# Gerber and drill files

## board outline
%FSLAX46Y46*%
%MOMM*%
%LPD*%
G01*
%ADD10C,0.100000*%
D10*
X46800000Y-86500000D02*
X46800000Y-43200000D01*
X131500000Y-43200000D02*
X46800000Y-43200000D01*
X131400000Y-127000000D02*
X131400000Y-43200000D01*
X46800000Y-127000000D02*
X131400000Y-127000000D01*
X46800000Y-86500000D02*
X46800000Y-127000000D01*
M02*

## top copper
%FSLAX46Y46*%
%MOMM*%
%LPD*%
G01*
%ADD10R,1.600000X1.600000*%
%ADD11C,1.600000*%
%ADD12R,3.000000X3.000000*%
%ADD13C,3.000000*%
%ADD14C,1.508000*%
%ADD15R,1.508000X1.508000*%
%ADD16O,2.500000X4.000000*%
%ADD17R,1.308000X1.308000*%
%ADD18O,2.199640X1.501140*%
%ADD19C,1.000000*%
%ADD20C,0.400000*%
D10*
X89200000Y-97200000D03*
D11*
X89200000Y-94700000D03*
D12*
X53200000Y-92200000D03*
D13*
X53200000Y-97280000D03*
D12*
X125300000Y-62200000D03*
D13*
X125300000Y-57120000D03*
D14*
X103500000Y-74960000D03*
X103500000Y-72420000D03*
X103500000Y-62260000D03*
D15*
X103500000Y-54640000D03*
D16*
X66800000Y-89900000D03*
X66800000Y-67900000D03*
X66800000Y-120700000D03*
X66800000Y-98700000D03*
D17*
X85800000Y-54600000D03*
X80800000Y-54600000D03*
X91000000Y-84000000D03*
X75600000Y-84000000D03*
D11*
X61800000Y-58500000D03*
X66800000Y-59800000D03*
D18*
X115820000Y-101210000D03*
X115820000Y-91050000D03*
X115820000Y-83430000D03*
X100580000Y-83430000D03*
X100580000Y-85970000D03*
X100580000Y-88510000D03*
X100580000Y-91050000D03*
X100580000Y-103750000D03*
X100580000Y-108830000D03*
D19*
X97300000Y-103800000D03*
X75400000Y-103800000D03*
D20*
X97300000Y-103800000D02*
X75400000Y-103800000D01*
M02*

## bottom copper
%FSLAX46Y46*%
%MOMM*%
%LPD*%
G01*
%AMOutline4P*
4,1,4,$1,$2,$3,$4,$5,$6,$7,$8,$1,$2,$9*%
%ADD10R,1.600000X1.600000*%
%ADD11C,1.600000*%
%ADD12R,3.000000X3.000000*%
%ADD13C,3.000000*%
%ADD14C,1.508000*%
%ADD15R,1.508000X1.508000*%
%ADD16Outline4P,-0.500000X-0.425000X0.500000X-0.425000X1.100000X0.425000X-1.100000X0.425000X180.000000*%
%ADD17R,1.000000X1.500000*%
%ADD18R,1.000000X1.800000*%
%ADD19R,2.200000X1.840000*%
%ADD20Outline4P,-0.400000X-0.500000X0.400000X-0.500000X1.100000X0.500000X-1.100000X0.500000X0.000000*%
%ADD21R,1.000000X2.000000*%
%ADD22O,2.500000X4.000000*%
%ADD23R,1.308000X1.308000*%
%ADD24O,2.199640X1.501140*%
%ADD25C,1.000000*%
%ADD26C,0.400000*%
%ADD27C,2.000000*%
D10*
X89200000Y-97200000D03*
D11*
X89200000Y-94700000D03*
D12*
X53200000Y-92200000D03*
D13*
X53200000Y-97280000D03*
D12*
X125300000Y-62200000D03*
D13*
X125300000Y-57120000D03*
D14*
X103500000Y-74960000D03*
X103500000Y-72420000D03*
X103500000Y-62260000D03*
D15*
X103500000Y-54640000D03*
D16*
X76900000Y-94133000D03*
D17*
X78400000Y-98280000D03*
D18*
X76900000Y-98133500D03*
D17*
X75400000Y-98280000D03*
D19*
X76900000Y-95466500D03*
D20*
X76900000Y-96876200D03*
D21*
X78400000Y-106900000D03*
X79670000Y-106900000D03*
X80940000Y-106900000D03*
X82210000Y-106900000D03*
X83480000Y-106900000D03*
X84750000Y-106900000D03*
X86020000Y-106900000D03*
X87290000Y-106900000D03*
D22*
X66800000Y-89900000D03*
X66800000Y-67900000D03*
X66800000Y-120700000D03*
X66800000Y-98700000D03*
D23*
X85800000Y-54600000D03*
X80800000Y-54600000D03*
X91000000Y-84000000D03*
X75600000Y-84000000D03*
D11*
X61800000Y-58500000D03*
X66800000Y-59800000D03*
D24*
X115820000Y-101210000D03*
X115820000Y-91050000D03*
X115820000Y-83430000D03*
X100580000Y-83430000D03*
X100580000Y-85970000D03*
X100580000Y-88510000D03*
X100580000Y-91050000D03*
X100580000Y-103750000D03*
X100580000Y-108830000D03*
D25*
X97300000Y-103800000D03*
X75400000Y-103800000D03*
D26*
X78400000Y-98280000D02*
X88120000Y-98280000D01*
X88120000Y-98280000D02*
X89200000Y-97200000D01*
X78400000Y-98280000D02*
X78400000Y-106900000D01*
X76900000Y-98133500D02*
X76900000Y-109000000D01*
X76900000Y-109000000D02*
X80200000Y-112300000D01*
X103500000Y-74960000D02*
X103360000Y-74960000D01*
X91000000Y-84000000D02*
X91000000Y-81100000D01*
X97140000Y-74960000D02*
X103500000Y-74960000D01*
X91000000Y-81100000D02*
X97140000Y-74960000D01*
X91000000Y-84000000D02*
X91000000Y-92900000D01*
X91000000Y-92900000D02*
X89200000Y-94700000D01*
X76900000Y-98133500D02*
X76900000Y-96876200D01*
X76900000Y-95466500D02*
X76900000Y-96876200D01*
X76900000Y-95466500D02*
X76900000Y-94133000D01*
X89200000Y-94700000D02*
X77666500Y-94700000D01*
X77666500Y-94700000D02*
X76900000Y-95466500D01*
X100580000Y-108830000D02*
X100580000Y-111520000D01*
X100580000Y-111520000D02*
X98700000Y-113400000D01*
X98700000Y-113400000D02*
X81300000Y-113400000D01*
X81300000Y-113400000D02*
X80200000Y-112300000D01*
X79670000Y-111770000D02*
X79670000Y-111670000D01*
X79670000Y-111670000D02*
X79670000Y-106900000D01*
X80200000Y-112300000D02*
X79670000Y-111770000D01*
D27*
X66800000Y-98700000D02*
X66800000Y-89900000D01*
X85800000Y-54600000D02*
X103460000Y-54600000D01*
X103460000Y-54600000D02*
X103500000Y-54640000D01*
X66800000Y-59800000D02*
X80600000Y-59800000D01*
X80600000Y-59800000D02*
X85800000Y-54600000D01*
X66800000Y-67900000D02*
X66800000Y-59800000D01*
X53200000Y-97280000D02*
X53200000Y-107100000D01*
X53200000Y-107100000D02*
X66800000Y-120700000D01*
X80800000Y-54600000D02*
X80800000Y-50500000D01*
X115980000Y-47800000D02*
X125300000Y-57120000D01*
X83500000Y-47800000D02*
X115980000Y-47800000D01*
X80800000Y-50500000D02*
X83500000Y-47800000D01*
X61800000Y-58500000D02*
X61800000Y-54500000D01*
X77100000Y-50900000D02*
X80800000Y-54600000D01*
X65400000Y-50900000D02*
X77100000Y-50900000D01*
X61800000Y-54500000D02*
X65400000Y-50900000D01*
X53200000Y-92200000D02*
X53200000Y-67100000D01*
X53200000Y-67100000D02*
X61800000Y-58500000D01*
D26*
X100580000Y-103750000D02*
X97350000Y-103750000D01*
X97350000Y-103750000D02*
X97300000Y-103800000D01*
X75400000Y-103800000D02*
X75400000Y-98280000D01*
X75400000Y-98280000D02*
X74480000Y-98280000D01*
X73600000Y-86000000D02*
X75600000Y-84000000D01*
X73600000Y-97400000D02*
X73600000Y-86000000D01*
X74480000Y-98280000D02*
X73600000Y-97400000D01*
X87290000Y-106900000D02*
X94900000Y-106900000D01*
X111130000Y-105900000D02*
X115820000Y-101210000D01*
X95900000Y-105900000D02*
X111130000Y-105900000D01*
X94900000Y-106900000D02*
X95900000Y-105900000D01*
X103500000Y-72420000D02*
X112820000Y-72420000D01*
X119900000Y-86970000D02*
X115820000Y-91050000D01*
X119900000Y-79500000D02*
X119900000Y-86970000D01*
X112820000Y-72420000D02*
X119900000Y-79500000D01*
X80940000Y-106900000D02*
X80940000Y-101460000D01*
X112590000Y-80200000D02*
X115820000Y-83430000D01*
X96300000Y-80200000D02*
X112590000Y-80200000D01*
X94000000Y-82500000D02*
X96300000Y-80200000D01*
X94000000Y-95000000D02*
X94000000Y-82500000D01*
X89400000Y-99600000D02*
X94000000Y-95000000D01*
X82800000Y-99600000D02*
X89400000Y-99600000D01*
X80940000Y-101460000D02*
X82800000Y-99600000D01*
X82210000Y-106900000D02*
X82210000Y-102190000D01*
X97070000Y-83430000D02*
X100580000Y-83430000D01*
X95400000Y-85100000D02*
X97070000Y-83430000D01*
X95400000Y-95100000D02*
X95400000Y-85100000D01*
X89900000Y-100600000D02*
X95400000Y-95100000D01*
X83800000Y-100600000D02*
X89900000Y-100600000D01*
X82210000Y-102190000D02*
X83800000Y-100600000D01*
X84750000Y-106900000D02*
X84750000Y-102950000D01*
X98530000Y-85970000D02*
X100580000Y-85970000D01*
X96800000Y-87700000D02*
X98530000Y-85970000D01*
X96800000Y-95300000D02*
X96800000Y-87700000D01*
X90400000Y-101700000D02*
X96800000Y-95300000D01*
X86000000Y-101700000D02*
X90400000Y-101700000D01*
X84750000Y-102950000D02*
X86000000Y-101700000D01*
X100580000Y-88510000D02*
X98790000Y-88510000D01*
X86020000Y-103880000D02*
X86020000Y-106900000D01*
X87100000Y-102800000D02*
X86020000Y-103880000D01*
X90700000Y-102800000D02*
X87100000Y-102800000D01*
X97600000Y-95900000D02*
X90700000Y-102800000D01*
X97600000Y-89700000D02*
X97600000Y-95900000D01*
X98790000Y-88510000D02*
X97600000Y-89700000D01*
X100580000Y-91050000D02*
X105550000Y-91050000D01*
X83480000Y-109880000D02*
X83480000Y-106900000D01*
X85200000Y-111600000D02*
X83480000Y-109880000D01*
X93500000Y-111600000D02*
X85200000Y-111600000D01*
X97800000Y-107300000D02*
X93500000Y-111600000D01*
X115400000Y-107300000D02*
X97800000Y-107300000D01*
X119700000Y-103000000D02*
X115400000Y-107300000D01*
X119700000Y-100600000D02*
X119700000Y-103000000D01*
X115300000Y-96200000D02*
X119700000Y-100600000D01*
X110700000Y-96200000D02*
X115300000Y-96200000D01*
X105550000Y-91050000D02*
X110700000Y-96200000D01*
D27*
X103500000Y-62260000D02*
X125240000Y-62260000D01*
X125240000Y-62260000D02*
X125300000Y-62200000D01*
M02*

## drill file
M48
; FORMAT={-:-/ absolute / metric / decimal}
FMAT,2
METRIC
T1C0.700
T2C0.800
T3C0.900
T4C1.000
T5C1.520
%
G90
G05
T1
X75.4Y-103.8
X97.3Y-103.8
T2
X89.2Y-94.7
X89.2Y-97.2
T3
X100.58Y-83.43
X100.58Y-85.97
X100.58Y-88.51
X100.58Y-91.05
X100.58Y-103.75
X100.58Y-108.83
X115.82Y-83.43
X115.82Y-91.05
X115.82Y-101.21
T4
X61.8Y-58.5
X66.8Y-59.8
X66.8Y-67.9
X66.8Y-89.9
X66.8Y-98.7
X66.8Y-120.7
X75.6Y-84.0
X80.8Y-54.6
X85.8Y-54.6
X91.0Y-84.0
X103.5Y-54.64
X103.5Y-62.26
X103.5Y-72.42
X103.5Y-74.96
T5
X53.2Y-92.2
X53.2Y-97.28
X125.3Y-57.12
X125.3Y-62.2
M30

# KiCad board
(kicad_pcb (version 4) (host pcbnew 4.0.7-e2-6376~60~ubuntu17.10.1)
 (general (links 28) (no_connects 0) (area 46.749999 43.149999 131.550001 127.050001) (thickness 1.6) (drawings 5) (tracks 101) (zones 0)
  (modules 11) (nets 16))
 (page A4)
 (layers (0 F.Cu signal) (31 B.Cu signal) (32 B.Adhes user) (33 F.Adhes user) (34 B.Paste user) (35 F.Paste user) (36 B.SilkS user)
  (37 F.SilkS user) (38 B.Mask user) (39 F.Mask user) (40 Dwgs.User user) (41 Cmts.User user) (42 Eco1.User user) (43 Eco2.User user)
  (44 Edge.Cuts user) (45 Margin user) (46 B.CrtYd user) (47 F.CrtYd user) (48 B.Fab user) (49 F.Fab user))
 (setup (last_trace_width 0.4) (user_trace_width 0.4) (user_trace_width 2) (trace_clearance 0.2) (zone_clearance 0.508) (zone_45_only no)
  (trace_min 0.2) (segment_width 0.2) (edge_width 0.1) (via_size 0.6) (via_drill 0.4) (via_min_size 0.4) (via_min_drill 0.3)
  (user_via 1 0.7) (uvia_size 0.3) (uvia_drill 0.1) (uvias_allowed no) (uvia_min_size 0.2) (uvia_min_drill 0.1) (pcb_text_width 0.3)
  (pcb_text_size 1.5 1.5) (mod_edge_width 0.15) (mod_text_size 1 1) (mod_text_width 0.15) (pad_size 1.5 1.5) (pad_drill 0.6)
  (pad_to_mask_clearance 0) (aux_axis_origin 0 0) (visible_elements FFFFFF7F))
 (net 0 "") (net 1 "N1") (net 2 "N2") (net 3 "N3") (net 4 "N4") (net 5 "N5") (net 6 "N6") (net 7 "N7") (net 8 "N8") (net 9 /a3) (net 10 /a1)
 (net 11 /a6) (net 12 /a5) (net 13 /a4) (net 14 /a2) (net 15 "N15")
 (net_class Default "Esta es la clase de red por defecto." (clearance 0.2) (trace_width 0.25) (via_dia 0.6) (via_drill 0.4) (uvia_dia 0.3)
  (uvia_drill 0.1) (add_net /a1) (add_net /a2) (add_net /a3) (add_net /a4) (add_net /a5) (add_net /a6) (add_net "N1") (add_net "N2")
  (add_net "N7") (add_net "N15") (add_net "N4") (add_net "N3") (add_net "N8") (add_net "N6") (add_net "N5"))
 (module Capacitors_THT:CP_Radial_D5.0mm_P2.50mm (layer F.Cu) (at 89.2 97.2 90)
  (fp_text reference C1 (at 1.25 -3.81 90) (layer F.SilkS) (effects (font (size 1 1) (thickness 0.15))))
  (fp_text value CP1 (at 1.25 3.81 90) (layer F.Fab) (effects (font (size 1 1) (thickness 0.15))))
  (pad 1 thru_hole rect (at 0 0 90) (size 1.6 1.6) (drill 0.8) (layers *.Cu *.Mask) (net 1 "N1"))
  (pad 2 thru_hole circle (at 2.5 0 90) (size 1.6 1.6) (drill 0.8) (layers *.Cu *.Mask) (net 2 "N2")))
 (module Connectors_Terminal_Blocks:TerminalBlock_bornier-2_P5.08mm (layer F.Cu) (at 53.2 92.2 270)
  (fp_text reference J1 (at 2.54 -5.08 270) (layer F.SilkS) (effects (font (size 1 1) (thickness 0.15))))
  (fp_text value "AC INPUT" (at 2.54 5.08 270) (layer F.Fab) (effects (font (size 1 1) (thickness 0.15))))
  (pad 1 thru_hole rect (at 0 0 270) (size 3 3) (drill 1.52) (layers *.Cu *.Mask) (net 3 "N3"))
  (pad 2 thru_hole circle (at 5.08 0 270) (size 3 3) (drill 1.52) (layers *.Cu *.Mask) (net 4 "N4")))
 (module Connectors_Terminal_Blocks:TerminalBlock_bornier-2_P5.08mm (layer F.Cu) (at 125.3 62.2 90)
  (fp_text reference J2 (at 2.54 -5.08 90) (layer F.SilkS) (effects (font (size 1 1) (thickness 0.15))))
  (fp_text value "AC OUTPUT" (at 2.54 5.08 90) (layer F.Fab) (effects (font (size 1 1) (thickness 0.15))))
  (pad 1 thru_hole rect (at 0 0 90) (size 3 3) (drill 1.52) (layers *.Cu *.Mask) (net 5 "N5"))
  (pad 2 thru_hole circle (at 5.08 0 90) (size 3 3) (drill 1.52) (layers *.Cu *.Mask) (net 3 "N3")))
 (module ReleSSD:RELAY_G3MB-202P (layer F.Cu) (at 102.1 64.8 90)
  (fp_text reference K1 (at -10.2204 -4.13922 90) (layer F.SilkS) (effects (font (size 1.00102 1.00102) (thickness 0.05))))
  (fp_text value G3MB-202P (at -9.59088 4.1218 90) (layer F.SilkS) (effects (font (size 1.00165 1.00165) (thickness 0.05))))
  (pad 4 thru_hole circle (at -10.16 1.4 90) (size 1.508 1.508) (drill 1) (layers *.Cu *.Mask F.SilkS) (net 2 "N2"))
  (pad 3 thru_hole circle (at -7.62 1.4 90) (size 1.508 1.508) (drill 1) (layers *.Cu *.Mask F.SilkS) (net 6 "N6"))
  (pad 2 thru_hole circle (at 2.54 1.4 90) (size 1.508 1.508) (drill 1) (layers *.Cu *.Mask F.SilkS) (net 5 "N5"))
  (pad 1 thru_hole rect (at 10.16 1.4 90) (size 1.508 1.508) (drill 1) (layers *.Cu *.Mask F.SilkS) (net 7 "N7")))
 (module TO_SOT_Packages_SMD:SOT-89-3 (layer B.Cu) (at 76.9 96.8 90)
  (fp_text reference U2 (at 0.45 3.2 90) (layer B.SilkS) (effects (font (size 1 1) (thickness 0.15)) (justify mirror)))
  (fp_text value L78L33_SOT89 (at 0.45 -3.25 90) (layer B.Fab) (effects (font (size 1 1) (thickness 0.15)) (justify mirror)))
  (pad 2 smd trapezoid (at 2.667 0 180) (size 1.6 0.85) (rect_delta 0 -0.6) (layers B.Cu B.Paste B.Mask) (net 2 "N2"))
  (pad 1 smd rect (at -1.48 1.5 180) (size 1 1.5) (layers B.Cu B.Paste B.Mask) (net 1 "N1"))
  (pad 2 smd rect (at -1.3335 0 180) (size 1 1.8) (layers B.Cu B.Paste B.Mask) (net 2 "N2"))
  (pad 3 smd rect (at -1.48 -1.5 180) (size 1 1.5) (layers B.Cu B.Paste B.Mask) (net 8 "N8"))
  (pad 2 smd rect (at 1.3335 0 180) (size 2.2 1.84) (layers B.Cu B.Paste B.Mask) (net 2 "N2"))
  (pad 2 smd trapezoid (at -0.0762 0) (size 1.5 1) (rect_delta 0 -0.7) (layers B.Cu B.Paste B.Mask) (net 2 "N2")))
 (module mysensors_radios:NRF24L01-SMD (layer B.Cu) (at 82.8 115.6)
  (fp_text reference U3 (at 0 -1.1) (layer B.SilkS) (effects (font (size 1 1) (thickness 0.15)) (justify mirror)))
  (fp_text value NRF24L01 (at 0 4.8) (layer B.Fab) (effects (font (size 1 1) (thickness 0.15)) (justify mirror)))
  (pad 2 smd rect (at -4.4 -8.7) (size 1 2) (layers B.Cu B.Paste B.Mask) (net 1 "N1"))
  (pad 1 smd rect (at -3.13 -8.7) (size 1 2) (layers B.Cu B.Paste B.Mask) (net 2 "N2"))
  (pad 3 smd rect (at -1.86 -8.7) (size 1 2) (layers B.Cu B.Paste B.Mask) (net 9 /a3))
  (pad 4 smd rect (at -0.59 -8.7) (size 1 2) (layers B.Cu B.Paste B.Mask) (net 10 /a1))
  (pad 5 smd rect (at 0.68 -8.7) (size 1 2) (layers B.Cu B.Paste B.Mask) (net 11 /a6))
  (pad 6 smd rect (at 1.95 -8.7) (size 1 2) (layers B.Cu B.Paste B.Mask) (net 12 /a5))
  (pad 7 smd rect (at 3.22 -8.7) (size 1 2) (layers B.Cu B.Paste B.Mask) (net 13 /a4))
  (pad 8 smd rect (at 4.49 -8.7) (size 1 2) (layers B.Cu B.Paste B.Mask) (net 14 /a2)))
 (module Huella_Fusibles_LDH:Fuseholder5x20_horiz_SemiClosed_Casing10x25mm (layer F.Cu) (at 66.8 67.9 270)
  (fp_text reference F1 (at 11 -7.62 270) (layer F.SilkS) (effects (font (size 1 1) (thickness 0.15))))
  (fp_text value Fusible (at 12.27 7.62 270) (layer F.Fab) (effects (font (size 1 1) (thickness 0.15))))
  (pad 2 thru_hole oval (at 22 0 180) (size 2.5 4) (drill 1) (layers *.Cu *.Mask) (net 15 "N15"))
  (pad 1 thru_hole oval (at 0 0 180) (size 2.5 4) (drill 1) (layers *.Cu *.Mask) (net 7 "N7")))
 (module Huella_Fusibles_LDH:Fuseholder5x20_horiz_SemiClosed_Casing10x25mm (layer F.Cu) (at 66.8 98.7 270)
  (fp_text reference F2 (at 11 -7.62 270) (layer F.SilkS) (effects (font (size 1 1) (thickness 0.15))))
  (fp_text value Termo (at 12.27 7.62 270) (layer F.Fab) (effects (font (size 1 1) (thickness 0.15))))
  (pad 2 thru_hole oval (at 22 0 180) (size 2.5 4) (drill 1) (layers *.Cu *.Mask) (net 4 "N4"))
  (pad 1 thru_hole oval (at 0 0 180) (size 2.5 4) (drill 1) (layers *.Cu *.Mask) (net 15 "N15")))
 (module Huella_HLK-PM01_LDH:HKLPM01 (layer F.Cu) (at 83.3 69.3 270)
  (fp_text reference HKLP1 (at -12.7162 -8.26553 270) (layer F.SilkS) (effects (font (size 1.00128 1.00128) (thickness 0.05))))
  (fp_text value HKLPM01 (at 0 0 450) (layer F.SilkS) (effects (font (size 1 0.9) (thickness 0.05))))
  (pad P$1 thru_hole rect (at -14.7 -2.5 270) (size 1.308 1.308) (drill 1) (layers *.Cu *.Mask F.SilkS) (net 7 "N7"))
  (pad P$2 thru_hole rect (at -14.7 2.5 270) (size 1.308 1.308) (drill 1) (layers *.Cu *.Mask F.SilkS) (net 3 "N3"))
  (pad P$3 thru_hole rect (at 14.7 -7.7 270) (size 1.308 1.308) (drill 1) (layers *.Cu *.Mask F.SilkS) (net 2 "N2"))
  (pad P$4 thru_hole rect (at 14.7 7.7 270) (size 1.308 1.308) (drill 1) (layers *.Cu *.Mask F.SilkS) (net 8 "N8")))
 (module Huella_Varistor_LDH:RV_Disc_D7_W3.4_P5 (layer F.Cu) (at 61.8 58.5)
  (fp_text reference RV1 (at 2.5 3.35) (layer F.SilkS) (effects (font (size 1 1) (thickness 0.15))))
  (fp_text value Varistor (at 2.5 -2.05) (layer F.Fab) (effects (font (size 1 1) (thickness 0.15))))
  (pad 1 thru_hole circle (at 0 0) (size 1.6 1.6) (drill 1) (layers *.Cu *.Mask) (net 3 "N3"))
  (pad 2 thru_hole circle (at 5 1.3) (size 1.6 1.6) (drill 1) (layers *.Cu *.Mask) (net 7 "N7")))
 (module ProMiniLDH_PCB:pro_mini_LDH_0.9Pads (layer F.Cu) (at 108.2 97.4 90)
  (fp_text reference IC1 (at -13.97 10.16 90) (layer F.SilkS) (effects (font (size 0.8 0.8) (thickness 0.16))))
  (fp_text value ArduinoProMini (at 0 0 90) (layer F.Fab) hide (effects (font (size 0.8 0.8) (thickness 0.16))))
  (pad 5 thru_hole oval (at -3.81 7.62 90) (size 1.50114 2.19964) (drill 0.9) (layers *.Cu *.Mask F.SilkS) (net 14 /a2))
  (pad 9 thru_hole oval (at 6.35 7.62 90) (size 1.50114 2.19964) (drill 0.9) (layers *.Cu *.Mask F.SilkS) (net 6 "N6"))
  (pad 12 thru_hole oval (at 13.97 7.62 90) (size 1.50114 2.19964) (drill 0.9) (layers *.Cu *.Mask F.SilkS) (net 9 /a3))
  (pad 13 thru_hole oval (at 13.97 -7.62 90) (size 1.50114 2.19964) (drill 0.9) (layers *.Cu *.Mask F.SilkS) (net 10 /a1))
  (pad 14 thru_hole oval (at 11.43 -7.62 90) (size 1.50114 2.19964) (drill 0.9) (layers *.Cu *.Mask F.SilkS) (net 12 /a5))
  (pad 15 thru_hole oval (at 8.89 -7.62 90) (size 1.50114 2.19964) (drill 0.9) (layers *.Cu *.Mask F.SilkS) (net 13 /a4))
  (pad 16 thru_hole oval (at 6.35 -7.62 90) (size 1.50114 2.19964) (drill 0.9) (layers *.Cu *.Mask F.SilkS) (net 11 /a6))
  (pad 21 thru_hole oval (at -6.35 -7.62 90) (size 1.50114 2.19964) (drill 0.9) (layers *.Cu *.Mask F.SilkS) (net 8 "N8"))
  (pad 23 thru_hole oval (at -11.43 -7.62 90) (size 1.50114 2.19964) (drill 0.9) (layers *.Cu *.Mask F.SilkS) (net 2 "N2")))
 (gr_line (start 46.8 86.5) (end 46.8 43.2) (angle 90) (layer Edge.Cuts) (width 0.1))
 (gr_line (start 131.5 43.2) (end 46.8 43.2) (angle 90) (layer Edge.Cuts) (width 0.1))
 (gr_line (start 131.4 127) (end 131.4 43.2) (angle 90) (layer Edge.Cuts) (width 0.1))
 (gr_line (start 46.8 127) (end 131.4 127) (angle 90) (layer Edge.Cuts) (width 0.1))
 (gr_line (start 46.8 86.5) (end 46.8 127) (angle 90) (layer Edge.Cuts) (width 0.1))
 (segment (start 78.4 98.28) (end 88.12 98.28) (width 0.4) (layer B.Cu) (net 1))
 (segment (start 88.12 98.28) (end 89.2 97.2) (width 0.4) (layer B.Cu) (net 1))
 (segment (start 78.4 98.28) (end 78.4 106.9) (width 0.4) (layer B.Cu) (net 1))
 (segment (start 76.9 98.1335) (end 76.9 109) (width 0.4) (layer B.Cu) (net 2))
 (segment (start 76.9 109) (end 80.2 112.3) (width 0.4) (layer B.Cu) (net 2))
 (segment (start 103.5 74.96) (end 103.36 74.96) (width 0.4) (layer B.Cu) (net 2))
 (segment (start 91 84) (end 91 81.1) (width 0.4) (layer B.Cu) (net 2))
 (segment (start 97.14 74.96) (end 103.5 74.96) (width 0.4) (layer B.Cu) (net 2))
 (segment (start 91 81.1) (end 97.14 74.96) (width 0.4) (layer B.Cu) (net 2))
 (segment (start 91 84) (end 91 92.9) (width 0.4) (layer B.Cu) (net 2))
 (segment (start 91 92.9) (end 89.2 94.7) (width 0.4) (layer B.Cu) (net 2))
 (segment (start 76.9 98.1335) (end 76.9 96.8762) (width 0.4) (layer B.Cu) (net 2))
 (segment (start 76.9 95.4665) (end 76.9 96.8762) (width 0.4) (layer B.Cu) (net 2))
 (segment (start 76.9 95.4665) (end 76.9 94.133) (width 0.4) (layer B.Cu) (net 2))
 (segment (start 89.2 94.7) (end 77.6665 94.7) (width 0.4) (layer B.Cu) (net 2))
 (segment (start 77.6665 94.7) (end 76.9 95.4665) (width 0.4) (layer B.Cu) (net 2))
 (segment (start 100.58 108.83) (end 100.58 111.52) (width 0.4) (layer B.Cu) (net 2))
 (segment (start 100.58 111.52) (end 98.7 113.4) (width 0.4) (layer B.Cu) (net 2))
 (segment (start 98.7 113.4) (end 81.3 113.4) (width 0.4) (layer B.Cu) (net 2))
 (segment (start 81.3 113.4) (end 80.2 112.3) (width 0.4) (layer B.Cu) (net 2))
 (segment (start 79.67 111.77) (end 79.67 111.67) (width 0.4) (layer B.Cu) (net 2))
 (segment (start 79.67 111.67) (end 79.67 106.9) (width 0.4) (layer B.Cu) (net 2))
 (segment (start 80.2 112.3) (end 79.67 111.77) (width 0.4) (layer B.Cu) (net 2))
 (segment (start 66.8 98.7) (end 66.8 89.9) (width 2) (layer B.Cu) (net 15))
 (segment (start 85.8 54.6) (end 103.46 54.6) (width 2) (layer B.Cu) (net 7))
 (segment (start 103.46 54.6) (end 103.5 54.64) (width 2) (layer B.Cu) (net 7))
 (segment (start 66.8 59.8) (end 80.6 59.8) (width 2) (layer B.Cu) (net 7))
 (segment (start 80.6 59.8) (end 85.8 54.6) (width 2) (layer B.Cu) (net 7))
 (segment (start 66.8 67.9) (end 66.8 59.8) (width 2) (layer B.Cu) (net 7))
 (segment (start 53.2 97.28) (end 53.2 107.1) (width 2) (layer B.Cu) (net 4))
 (segment (start 53.2 107.1) (end 66.8 120.7) (width 2) (layer B.Cu) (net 4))
 (segment (start 80.8 54.6) (end 80.8 50.5) (width 2) (layer B.Cu) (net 3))
 (segment (start 115.98 47.8) (end 125.3 57.12) (width 2) (layer B.Cu) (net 3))
 (segment (start 83.5 47.8) (end 115.98 47.8) (width 2) (layer B.Cu) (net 3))
 (segment (start 80.8 50.5) (end 83.5 47.8) (width 2) (layer B.Cu) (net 3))
 (segment (start 61.8 58.5) (end 61.8 54.5) (width 2) (layer B.Cu) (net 3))
 (segment (start 77.1 50.9) (end 80.8 54.6) (width 2) (layer B.Cu) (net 3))
 (segment (start 65.4 50.9) (end 77.1 50.9) (width 2) (layer B.Cu) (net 3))
 (segment (start 61.8 54.5) (end 65.4 50.9) (width 2) (layer B.Cu) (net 3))
 (segment (start 53.2 92.2) (end 53.2 67.1) (width 2) (layer B.Cu) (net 3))
 (segment (start 53.2 67.1) (end 61.8 58.5) (width 2) (layer B.Cu) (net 3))
 (segment (start 100.58 103.75) (end 97.35 103.75) (width 0.4) (layer B.Cu) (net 8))
 (segment (start 97.35 103.75) (end 97.3 103.8) (width 0.4) (layer B.Cu) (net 8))
 (via (at 97.3 103.8) (size 1) (drill 0.7) (layers F.Cu B.Cu) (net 8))
 (segment (start 97.3 103.8) (end 75.4 103.8) (width 0.4) (layer F.Cu) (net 8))
 (via (at 75.4 103.8) (size 1) (drill 0.7) (layers F.Cu B.Cu) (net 8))
 (segment (start 75.4 103.8) (end 75.4 98.28) (width 0.4) (layer B.Cu) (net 8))
 (segment (start 75.4 98.28) (end 74.48 98.28) (width 0.4) (layer B.Cu) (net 8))
 (segment (start 73.6 86) (end 75.6 84) (width 0.4) (layer B.Cu) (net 8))
 (segment (start 73.6 97.4) (end 73.6 86) (width 0.4) (layer B.Cu) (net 8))
 (segment (start 74.48 98.28) (end 73.6 97.4) (width 0.4) (layer B.Cu) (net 8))
 (segment (start 87.29 106.9) (end 94.9 106.9) (width 0.4) (layer B.Cu) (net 14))
 (segment (start 111.13 105.9) (end 115.82 101.21) (width 0.4) (layer B.Cu) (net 14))
 (segment (start 95.9 105.9) (end 111.13 105.9) (width 0.4) (layer B.Cu) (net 14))
 (segment (start 94.9 106.9) (end 95.9 105.9) (width 0.4) (layer B.Cu) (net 14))
 (segment (start 103.5 72.42) (end 112.82 72.42) (width 0.4) (layer B.Cu) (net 6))
 (segment (start 119.9 86.97) (end 115.82 91.05) (width 0.4) (layer B.Cu) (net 6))
 (segment (start 119.9 79.5) (end 119.9 86.97) (width 0.4) (layer B.Cu) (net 6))
 (segment (start 112.82 72.42) (end 119.9 79.5) (width 0.4) (layer B.Cu) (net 6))
 (segment (start 80.94 106.9) (end 80.94 101.46) (width 0.4) (layer B.Cu) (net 9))
 (segment (start 112.59 80.2) (end 115.82 83.43) (width 0.4) (layer B.Cu) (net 9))
 (segment (start 96.3 80.2) (end 112.59 80.2) (width 0.4) (layer B.Cu) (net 9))
 (segment (start 94 82.5) (end 96.3 80.2) (width 0.4) (layer B.Cu) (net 9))
 (segment (start 94 95) (end 94 82.5) (width 0.4) (layer B.Cu) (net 9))
 (segment (start 89.4 99.6) (end 94 95) (width 0.4) (layer B.Cu) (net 9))
 (segment (start 82.8 99.6) (end 89.4 99.6) (width 0.4) (layer B.Cu) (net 9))
 (segment (start 80.94 101.46) (end 82.8 99.6) (width 0.4) (layer B.Cu) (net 9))
 (segment (start 82.21 106.9) (end 82.21 102.19) (width 0.4) (layer B.Cu) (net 10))
 (segment (start 97.07 83.43) (end 100.58 83.43) (width 0.4) (layer B.Cu) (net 10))
 (segment (start 95.4 85.1) (end 97.07 83.43) (width 0.4) (layer B.Cu) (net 10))
 (segment (start 95.4 95.1) (end 95.4 85.1) (width 0.4) (layer B.Cu) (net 10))
 (segment (start 89.9 100.6) (end 95.4 95.1) (width 0.4) (layer B.Cu) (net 10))
 (segment (start 83.8 100.6) (end 89.9 100.6) (width 0.4) (layer B.Cu) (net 10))
 (segment (start 82.21 102.19) (end 83.8 100.6) (width 0.4) (layer B.Cu) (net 10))
 (segment (start 84.75 106.9) (end 84.75 102.95) (width 0.4) (layer B.Cu) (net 12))
 (segment (start 98.53 85.97) (end 100.58 85.97) (width 0.4) (layer B.Cu) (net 12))
 (segment (start 96.8 87.7) (end 98.53 85.97) (width 0.4) (layer B.Cu) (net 12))
 (segment (start 96.8 95.3) (end 96.8 87.7) (width 0.4) (layer B.Cu) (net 12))
 (segment (start 90.4 101.7) (end 96.8 95.3) (width 0.4) (layer B.Cu) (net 12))
 (segment (start 86 101.7) (end 90.4 101.7) (width 0.4) (layer B.Cu) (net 12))
 (segment (start 84.75 102.95) (end 86 101.7) (width 0.4) (layer B.Cu) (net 12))
 (segment (start 100.58 88.51) (end 98.79 88.51) (width 0.4) (layer B.Cu) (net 13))
 (segment (start 86.02 103.88) (end 86.02 106.9) (width 0.4) (layer B.Cu) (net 13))
 (segment (start 87.1 102.8) (end 86.02 103.88) (width 0.4) (layer B.Cu) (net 13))
 (segment (start 90.7 102.8) (end 87.1 102.8) (width 0.4) (layer B.Cu) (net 13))
 (segment (start 97.6 95.9) (end 90.7 102.8) (width 0.4) (layer B.Cu) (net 13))
 (segment (start 97.6 89.7) (end 97.6 95.9) (width 0.4) (layer B.Cu) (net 13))
 (segment (start 98.79 88.51) (end 97.6 89.7) (width 0.4) (layer B.Cu) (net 13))
 (segment (start 100.58 91.05) (end 105.55 91.05) (width 0.4) (layer B.Cu) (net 11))
 (segment (start 83.48 109.88) (end 83.48 106.9) (width 0.4) (layer B.Cu) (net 11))
 (segment (start 85.2 111.6) (end 83.48 109.88) (width 0.4) (layer B.Cu) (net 11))
 (segment (start 93.5 111.6) (end 85.2 111.6) (width 0.4) (layer B.Cu) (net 11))
 (segment (start 97.8 107.3) (end 93.5 111.6) (width 0.4) (layer B.Cu) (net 11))
 (segment (start 115.4 107.3) (end 97.8 107.3) (width 0.4) (layer B.Cu) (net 11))
 (segment (start 119.7 103) (end 115.4 107.3) (width 0.4) (layer B.Cu) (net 11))
 (segment (start 119.7 100.6) (end 119.7 103) (width 0.4) (layer B.Cu) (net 11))
 (segment (start 115.3 96.2) (end 119.7 100.6) (width 0.4) (layer B.Cu) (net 11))
 (segment (start 110.7 96.2) (end 115.3 96.2) (width 0.4) (layer B.Cu) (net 11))
 (segment (start 105.55 91.05) (end 110.7 96.2) (width 0.4) (layer B.Cu) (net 11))
 (segment (start 103.5 62.26) (end 125.24 62.26) (width 2) (layer B.Cu) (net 5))
 (segment (start 125.24 62.26) (end 125.3 62.2) (width 2) (layer B.Cu) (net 5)))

